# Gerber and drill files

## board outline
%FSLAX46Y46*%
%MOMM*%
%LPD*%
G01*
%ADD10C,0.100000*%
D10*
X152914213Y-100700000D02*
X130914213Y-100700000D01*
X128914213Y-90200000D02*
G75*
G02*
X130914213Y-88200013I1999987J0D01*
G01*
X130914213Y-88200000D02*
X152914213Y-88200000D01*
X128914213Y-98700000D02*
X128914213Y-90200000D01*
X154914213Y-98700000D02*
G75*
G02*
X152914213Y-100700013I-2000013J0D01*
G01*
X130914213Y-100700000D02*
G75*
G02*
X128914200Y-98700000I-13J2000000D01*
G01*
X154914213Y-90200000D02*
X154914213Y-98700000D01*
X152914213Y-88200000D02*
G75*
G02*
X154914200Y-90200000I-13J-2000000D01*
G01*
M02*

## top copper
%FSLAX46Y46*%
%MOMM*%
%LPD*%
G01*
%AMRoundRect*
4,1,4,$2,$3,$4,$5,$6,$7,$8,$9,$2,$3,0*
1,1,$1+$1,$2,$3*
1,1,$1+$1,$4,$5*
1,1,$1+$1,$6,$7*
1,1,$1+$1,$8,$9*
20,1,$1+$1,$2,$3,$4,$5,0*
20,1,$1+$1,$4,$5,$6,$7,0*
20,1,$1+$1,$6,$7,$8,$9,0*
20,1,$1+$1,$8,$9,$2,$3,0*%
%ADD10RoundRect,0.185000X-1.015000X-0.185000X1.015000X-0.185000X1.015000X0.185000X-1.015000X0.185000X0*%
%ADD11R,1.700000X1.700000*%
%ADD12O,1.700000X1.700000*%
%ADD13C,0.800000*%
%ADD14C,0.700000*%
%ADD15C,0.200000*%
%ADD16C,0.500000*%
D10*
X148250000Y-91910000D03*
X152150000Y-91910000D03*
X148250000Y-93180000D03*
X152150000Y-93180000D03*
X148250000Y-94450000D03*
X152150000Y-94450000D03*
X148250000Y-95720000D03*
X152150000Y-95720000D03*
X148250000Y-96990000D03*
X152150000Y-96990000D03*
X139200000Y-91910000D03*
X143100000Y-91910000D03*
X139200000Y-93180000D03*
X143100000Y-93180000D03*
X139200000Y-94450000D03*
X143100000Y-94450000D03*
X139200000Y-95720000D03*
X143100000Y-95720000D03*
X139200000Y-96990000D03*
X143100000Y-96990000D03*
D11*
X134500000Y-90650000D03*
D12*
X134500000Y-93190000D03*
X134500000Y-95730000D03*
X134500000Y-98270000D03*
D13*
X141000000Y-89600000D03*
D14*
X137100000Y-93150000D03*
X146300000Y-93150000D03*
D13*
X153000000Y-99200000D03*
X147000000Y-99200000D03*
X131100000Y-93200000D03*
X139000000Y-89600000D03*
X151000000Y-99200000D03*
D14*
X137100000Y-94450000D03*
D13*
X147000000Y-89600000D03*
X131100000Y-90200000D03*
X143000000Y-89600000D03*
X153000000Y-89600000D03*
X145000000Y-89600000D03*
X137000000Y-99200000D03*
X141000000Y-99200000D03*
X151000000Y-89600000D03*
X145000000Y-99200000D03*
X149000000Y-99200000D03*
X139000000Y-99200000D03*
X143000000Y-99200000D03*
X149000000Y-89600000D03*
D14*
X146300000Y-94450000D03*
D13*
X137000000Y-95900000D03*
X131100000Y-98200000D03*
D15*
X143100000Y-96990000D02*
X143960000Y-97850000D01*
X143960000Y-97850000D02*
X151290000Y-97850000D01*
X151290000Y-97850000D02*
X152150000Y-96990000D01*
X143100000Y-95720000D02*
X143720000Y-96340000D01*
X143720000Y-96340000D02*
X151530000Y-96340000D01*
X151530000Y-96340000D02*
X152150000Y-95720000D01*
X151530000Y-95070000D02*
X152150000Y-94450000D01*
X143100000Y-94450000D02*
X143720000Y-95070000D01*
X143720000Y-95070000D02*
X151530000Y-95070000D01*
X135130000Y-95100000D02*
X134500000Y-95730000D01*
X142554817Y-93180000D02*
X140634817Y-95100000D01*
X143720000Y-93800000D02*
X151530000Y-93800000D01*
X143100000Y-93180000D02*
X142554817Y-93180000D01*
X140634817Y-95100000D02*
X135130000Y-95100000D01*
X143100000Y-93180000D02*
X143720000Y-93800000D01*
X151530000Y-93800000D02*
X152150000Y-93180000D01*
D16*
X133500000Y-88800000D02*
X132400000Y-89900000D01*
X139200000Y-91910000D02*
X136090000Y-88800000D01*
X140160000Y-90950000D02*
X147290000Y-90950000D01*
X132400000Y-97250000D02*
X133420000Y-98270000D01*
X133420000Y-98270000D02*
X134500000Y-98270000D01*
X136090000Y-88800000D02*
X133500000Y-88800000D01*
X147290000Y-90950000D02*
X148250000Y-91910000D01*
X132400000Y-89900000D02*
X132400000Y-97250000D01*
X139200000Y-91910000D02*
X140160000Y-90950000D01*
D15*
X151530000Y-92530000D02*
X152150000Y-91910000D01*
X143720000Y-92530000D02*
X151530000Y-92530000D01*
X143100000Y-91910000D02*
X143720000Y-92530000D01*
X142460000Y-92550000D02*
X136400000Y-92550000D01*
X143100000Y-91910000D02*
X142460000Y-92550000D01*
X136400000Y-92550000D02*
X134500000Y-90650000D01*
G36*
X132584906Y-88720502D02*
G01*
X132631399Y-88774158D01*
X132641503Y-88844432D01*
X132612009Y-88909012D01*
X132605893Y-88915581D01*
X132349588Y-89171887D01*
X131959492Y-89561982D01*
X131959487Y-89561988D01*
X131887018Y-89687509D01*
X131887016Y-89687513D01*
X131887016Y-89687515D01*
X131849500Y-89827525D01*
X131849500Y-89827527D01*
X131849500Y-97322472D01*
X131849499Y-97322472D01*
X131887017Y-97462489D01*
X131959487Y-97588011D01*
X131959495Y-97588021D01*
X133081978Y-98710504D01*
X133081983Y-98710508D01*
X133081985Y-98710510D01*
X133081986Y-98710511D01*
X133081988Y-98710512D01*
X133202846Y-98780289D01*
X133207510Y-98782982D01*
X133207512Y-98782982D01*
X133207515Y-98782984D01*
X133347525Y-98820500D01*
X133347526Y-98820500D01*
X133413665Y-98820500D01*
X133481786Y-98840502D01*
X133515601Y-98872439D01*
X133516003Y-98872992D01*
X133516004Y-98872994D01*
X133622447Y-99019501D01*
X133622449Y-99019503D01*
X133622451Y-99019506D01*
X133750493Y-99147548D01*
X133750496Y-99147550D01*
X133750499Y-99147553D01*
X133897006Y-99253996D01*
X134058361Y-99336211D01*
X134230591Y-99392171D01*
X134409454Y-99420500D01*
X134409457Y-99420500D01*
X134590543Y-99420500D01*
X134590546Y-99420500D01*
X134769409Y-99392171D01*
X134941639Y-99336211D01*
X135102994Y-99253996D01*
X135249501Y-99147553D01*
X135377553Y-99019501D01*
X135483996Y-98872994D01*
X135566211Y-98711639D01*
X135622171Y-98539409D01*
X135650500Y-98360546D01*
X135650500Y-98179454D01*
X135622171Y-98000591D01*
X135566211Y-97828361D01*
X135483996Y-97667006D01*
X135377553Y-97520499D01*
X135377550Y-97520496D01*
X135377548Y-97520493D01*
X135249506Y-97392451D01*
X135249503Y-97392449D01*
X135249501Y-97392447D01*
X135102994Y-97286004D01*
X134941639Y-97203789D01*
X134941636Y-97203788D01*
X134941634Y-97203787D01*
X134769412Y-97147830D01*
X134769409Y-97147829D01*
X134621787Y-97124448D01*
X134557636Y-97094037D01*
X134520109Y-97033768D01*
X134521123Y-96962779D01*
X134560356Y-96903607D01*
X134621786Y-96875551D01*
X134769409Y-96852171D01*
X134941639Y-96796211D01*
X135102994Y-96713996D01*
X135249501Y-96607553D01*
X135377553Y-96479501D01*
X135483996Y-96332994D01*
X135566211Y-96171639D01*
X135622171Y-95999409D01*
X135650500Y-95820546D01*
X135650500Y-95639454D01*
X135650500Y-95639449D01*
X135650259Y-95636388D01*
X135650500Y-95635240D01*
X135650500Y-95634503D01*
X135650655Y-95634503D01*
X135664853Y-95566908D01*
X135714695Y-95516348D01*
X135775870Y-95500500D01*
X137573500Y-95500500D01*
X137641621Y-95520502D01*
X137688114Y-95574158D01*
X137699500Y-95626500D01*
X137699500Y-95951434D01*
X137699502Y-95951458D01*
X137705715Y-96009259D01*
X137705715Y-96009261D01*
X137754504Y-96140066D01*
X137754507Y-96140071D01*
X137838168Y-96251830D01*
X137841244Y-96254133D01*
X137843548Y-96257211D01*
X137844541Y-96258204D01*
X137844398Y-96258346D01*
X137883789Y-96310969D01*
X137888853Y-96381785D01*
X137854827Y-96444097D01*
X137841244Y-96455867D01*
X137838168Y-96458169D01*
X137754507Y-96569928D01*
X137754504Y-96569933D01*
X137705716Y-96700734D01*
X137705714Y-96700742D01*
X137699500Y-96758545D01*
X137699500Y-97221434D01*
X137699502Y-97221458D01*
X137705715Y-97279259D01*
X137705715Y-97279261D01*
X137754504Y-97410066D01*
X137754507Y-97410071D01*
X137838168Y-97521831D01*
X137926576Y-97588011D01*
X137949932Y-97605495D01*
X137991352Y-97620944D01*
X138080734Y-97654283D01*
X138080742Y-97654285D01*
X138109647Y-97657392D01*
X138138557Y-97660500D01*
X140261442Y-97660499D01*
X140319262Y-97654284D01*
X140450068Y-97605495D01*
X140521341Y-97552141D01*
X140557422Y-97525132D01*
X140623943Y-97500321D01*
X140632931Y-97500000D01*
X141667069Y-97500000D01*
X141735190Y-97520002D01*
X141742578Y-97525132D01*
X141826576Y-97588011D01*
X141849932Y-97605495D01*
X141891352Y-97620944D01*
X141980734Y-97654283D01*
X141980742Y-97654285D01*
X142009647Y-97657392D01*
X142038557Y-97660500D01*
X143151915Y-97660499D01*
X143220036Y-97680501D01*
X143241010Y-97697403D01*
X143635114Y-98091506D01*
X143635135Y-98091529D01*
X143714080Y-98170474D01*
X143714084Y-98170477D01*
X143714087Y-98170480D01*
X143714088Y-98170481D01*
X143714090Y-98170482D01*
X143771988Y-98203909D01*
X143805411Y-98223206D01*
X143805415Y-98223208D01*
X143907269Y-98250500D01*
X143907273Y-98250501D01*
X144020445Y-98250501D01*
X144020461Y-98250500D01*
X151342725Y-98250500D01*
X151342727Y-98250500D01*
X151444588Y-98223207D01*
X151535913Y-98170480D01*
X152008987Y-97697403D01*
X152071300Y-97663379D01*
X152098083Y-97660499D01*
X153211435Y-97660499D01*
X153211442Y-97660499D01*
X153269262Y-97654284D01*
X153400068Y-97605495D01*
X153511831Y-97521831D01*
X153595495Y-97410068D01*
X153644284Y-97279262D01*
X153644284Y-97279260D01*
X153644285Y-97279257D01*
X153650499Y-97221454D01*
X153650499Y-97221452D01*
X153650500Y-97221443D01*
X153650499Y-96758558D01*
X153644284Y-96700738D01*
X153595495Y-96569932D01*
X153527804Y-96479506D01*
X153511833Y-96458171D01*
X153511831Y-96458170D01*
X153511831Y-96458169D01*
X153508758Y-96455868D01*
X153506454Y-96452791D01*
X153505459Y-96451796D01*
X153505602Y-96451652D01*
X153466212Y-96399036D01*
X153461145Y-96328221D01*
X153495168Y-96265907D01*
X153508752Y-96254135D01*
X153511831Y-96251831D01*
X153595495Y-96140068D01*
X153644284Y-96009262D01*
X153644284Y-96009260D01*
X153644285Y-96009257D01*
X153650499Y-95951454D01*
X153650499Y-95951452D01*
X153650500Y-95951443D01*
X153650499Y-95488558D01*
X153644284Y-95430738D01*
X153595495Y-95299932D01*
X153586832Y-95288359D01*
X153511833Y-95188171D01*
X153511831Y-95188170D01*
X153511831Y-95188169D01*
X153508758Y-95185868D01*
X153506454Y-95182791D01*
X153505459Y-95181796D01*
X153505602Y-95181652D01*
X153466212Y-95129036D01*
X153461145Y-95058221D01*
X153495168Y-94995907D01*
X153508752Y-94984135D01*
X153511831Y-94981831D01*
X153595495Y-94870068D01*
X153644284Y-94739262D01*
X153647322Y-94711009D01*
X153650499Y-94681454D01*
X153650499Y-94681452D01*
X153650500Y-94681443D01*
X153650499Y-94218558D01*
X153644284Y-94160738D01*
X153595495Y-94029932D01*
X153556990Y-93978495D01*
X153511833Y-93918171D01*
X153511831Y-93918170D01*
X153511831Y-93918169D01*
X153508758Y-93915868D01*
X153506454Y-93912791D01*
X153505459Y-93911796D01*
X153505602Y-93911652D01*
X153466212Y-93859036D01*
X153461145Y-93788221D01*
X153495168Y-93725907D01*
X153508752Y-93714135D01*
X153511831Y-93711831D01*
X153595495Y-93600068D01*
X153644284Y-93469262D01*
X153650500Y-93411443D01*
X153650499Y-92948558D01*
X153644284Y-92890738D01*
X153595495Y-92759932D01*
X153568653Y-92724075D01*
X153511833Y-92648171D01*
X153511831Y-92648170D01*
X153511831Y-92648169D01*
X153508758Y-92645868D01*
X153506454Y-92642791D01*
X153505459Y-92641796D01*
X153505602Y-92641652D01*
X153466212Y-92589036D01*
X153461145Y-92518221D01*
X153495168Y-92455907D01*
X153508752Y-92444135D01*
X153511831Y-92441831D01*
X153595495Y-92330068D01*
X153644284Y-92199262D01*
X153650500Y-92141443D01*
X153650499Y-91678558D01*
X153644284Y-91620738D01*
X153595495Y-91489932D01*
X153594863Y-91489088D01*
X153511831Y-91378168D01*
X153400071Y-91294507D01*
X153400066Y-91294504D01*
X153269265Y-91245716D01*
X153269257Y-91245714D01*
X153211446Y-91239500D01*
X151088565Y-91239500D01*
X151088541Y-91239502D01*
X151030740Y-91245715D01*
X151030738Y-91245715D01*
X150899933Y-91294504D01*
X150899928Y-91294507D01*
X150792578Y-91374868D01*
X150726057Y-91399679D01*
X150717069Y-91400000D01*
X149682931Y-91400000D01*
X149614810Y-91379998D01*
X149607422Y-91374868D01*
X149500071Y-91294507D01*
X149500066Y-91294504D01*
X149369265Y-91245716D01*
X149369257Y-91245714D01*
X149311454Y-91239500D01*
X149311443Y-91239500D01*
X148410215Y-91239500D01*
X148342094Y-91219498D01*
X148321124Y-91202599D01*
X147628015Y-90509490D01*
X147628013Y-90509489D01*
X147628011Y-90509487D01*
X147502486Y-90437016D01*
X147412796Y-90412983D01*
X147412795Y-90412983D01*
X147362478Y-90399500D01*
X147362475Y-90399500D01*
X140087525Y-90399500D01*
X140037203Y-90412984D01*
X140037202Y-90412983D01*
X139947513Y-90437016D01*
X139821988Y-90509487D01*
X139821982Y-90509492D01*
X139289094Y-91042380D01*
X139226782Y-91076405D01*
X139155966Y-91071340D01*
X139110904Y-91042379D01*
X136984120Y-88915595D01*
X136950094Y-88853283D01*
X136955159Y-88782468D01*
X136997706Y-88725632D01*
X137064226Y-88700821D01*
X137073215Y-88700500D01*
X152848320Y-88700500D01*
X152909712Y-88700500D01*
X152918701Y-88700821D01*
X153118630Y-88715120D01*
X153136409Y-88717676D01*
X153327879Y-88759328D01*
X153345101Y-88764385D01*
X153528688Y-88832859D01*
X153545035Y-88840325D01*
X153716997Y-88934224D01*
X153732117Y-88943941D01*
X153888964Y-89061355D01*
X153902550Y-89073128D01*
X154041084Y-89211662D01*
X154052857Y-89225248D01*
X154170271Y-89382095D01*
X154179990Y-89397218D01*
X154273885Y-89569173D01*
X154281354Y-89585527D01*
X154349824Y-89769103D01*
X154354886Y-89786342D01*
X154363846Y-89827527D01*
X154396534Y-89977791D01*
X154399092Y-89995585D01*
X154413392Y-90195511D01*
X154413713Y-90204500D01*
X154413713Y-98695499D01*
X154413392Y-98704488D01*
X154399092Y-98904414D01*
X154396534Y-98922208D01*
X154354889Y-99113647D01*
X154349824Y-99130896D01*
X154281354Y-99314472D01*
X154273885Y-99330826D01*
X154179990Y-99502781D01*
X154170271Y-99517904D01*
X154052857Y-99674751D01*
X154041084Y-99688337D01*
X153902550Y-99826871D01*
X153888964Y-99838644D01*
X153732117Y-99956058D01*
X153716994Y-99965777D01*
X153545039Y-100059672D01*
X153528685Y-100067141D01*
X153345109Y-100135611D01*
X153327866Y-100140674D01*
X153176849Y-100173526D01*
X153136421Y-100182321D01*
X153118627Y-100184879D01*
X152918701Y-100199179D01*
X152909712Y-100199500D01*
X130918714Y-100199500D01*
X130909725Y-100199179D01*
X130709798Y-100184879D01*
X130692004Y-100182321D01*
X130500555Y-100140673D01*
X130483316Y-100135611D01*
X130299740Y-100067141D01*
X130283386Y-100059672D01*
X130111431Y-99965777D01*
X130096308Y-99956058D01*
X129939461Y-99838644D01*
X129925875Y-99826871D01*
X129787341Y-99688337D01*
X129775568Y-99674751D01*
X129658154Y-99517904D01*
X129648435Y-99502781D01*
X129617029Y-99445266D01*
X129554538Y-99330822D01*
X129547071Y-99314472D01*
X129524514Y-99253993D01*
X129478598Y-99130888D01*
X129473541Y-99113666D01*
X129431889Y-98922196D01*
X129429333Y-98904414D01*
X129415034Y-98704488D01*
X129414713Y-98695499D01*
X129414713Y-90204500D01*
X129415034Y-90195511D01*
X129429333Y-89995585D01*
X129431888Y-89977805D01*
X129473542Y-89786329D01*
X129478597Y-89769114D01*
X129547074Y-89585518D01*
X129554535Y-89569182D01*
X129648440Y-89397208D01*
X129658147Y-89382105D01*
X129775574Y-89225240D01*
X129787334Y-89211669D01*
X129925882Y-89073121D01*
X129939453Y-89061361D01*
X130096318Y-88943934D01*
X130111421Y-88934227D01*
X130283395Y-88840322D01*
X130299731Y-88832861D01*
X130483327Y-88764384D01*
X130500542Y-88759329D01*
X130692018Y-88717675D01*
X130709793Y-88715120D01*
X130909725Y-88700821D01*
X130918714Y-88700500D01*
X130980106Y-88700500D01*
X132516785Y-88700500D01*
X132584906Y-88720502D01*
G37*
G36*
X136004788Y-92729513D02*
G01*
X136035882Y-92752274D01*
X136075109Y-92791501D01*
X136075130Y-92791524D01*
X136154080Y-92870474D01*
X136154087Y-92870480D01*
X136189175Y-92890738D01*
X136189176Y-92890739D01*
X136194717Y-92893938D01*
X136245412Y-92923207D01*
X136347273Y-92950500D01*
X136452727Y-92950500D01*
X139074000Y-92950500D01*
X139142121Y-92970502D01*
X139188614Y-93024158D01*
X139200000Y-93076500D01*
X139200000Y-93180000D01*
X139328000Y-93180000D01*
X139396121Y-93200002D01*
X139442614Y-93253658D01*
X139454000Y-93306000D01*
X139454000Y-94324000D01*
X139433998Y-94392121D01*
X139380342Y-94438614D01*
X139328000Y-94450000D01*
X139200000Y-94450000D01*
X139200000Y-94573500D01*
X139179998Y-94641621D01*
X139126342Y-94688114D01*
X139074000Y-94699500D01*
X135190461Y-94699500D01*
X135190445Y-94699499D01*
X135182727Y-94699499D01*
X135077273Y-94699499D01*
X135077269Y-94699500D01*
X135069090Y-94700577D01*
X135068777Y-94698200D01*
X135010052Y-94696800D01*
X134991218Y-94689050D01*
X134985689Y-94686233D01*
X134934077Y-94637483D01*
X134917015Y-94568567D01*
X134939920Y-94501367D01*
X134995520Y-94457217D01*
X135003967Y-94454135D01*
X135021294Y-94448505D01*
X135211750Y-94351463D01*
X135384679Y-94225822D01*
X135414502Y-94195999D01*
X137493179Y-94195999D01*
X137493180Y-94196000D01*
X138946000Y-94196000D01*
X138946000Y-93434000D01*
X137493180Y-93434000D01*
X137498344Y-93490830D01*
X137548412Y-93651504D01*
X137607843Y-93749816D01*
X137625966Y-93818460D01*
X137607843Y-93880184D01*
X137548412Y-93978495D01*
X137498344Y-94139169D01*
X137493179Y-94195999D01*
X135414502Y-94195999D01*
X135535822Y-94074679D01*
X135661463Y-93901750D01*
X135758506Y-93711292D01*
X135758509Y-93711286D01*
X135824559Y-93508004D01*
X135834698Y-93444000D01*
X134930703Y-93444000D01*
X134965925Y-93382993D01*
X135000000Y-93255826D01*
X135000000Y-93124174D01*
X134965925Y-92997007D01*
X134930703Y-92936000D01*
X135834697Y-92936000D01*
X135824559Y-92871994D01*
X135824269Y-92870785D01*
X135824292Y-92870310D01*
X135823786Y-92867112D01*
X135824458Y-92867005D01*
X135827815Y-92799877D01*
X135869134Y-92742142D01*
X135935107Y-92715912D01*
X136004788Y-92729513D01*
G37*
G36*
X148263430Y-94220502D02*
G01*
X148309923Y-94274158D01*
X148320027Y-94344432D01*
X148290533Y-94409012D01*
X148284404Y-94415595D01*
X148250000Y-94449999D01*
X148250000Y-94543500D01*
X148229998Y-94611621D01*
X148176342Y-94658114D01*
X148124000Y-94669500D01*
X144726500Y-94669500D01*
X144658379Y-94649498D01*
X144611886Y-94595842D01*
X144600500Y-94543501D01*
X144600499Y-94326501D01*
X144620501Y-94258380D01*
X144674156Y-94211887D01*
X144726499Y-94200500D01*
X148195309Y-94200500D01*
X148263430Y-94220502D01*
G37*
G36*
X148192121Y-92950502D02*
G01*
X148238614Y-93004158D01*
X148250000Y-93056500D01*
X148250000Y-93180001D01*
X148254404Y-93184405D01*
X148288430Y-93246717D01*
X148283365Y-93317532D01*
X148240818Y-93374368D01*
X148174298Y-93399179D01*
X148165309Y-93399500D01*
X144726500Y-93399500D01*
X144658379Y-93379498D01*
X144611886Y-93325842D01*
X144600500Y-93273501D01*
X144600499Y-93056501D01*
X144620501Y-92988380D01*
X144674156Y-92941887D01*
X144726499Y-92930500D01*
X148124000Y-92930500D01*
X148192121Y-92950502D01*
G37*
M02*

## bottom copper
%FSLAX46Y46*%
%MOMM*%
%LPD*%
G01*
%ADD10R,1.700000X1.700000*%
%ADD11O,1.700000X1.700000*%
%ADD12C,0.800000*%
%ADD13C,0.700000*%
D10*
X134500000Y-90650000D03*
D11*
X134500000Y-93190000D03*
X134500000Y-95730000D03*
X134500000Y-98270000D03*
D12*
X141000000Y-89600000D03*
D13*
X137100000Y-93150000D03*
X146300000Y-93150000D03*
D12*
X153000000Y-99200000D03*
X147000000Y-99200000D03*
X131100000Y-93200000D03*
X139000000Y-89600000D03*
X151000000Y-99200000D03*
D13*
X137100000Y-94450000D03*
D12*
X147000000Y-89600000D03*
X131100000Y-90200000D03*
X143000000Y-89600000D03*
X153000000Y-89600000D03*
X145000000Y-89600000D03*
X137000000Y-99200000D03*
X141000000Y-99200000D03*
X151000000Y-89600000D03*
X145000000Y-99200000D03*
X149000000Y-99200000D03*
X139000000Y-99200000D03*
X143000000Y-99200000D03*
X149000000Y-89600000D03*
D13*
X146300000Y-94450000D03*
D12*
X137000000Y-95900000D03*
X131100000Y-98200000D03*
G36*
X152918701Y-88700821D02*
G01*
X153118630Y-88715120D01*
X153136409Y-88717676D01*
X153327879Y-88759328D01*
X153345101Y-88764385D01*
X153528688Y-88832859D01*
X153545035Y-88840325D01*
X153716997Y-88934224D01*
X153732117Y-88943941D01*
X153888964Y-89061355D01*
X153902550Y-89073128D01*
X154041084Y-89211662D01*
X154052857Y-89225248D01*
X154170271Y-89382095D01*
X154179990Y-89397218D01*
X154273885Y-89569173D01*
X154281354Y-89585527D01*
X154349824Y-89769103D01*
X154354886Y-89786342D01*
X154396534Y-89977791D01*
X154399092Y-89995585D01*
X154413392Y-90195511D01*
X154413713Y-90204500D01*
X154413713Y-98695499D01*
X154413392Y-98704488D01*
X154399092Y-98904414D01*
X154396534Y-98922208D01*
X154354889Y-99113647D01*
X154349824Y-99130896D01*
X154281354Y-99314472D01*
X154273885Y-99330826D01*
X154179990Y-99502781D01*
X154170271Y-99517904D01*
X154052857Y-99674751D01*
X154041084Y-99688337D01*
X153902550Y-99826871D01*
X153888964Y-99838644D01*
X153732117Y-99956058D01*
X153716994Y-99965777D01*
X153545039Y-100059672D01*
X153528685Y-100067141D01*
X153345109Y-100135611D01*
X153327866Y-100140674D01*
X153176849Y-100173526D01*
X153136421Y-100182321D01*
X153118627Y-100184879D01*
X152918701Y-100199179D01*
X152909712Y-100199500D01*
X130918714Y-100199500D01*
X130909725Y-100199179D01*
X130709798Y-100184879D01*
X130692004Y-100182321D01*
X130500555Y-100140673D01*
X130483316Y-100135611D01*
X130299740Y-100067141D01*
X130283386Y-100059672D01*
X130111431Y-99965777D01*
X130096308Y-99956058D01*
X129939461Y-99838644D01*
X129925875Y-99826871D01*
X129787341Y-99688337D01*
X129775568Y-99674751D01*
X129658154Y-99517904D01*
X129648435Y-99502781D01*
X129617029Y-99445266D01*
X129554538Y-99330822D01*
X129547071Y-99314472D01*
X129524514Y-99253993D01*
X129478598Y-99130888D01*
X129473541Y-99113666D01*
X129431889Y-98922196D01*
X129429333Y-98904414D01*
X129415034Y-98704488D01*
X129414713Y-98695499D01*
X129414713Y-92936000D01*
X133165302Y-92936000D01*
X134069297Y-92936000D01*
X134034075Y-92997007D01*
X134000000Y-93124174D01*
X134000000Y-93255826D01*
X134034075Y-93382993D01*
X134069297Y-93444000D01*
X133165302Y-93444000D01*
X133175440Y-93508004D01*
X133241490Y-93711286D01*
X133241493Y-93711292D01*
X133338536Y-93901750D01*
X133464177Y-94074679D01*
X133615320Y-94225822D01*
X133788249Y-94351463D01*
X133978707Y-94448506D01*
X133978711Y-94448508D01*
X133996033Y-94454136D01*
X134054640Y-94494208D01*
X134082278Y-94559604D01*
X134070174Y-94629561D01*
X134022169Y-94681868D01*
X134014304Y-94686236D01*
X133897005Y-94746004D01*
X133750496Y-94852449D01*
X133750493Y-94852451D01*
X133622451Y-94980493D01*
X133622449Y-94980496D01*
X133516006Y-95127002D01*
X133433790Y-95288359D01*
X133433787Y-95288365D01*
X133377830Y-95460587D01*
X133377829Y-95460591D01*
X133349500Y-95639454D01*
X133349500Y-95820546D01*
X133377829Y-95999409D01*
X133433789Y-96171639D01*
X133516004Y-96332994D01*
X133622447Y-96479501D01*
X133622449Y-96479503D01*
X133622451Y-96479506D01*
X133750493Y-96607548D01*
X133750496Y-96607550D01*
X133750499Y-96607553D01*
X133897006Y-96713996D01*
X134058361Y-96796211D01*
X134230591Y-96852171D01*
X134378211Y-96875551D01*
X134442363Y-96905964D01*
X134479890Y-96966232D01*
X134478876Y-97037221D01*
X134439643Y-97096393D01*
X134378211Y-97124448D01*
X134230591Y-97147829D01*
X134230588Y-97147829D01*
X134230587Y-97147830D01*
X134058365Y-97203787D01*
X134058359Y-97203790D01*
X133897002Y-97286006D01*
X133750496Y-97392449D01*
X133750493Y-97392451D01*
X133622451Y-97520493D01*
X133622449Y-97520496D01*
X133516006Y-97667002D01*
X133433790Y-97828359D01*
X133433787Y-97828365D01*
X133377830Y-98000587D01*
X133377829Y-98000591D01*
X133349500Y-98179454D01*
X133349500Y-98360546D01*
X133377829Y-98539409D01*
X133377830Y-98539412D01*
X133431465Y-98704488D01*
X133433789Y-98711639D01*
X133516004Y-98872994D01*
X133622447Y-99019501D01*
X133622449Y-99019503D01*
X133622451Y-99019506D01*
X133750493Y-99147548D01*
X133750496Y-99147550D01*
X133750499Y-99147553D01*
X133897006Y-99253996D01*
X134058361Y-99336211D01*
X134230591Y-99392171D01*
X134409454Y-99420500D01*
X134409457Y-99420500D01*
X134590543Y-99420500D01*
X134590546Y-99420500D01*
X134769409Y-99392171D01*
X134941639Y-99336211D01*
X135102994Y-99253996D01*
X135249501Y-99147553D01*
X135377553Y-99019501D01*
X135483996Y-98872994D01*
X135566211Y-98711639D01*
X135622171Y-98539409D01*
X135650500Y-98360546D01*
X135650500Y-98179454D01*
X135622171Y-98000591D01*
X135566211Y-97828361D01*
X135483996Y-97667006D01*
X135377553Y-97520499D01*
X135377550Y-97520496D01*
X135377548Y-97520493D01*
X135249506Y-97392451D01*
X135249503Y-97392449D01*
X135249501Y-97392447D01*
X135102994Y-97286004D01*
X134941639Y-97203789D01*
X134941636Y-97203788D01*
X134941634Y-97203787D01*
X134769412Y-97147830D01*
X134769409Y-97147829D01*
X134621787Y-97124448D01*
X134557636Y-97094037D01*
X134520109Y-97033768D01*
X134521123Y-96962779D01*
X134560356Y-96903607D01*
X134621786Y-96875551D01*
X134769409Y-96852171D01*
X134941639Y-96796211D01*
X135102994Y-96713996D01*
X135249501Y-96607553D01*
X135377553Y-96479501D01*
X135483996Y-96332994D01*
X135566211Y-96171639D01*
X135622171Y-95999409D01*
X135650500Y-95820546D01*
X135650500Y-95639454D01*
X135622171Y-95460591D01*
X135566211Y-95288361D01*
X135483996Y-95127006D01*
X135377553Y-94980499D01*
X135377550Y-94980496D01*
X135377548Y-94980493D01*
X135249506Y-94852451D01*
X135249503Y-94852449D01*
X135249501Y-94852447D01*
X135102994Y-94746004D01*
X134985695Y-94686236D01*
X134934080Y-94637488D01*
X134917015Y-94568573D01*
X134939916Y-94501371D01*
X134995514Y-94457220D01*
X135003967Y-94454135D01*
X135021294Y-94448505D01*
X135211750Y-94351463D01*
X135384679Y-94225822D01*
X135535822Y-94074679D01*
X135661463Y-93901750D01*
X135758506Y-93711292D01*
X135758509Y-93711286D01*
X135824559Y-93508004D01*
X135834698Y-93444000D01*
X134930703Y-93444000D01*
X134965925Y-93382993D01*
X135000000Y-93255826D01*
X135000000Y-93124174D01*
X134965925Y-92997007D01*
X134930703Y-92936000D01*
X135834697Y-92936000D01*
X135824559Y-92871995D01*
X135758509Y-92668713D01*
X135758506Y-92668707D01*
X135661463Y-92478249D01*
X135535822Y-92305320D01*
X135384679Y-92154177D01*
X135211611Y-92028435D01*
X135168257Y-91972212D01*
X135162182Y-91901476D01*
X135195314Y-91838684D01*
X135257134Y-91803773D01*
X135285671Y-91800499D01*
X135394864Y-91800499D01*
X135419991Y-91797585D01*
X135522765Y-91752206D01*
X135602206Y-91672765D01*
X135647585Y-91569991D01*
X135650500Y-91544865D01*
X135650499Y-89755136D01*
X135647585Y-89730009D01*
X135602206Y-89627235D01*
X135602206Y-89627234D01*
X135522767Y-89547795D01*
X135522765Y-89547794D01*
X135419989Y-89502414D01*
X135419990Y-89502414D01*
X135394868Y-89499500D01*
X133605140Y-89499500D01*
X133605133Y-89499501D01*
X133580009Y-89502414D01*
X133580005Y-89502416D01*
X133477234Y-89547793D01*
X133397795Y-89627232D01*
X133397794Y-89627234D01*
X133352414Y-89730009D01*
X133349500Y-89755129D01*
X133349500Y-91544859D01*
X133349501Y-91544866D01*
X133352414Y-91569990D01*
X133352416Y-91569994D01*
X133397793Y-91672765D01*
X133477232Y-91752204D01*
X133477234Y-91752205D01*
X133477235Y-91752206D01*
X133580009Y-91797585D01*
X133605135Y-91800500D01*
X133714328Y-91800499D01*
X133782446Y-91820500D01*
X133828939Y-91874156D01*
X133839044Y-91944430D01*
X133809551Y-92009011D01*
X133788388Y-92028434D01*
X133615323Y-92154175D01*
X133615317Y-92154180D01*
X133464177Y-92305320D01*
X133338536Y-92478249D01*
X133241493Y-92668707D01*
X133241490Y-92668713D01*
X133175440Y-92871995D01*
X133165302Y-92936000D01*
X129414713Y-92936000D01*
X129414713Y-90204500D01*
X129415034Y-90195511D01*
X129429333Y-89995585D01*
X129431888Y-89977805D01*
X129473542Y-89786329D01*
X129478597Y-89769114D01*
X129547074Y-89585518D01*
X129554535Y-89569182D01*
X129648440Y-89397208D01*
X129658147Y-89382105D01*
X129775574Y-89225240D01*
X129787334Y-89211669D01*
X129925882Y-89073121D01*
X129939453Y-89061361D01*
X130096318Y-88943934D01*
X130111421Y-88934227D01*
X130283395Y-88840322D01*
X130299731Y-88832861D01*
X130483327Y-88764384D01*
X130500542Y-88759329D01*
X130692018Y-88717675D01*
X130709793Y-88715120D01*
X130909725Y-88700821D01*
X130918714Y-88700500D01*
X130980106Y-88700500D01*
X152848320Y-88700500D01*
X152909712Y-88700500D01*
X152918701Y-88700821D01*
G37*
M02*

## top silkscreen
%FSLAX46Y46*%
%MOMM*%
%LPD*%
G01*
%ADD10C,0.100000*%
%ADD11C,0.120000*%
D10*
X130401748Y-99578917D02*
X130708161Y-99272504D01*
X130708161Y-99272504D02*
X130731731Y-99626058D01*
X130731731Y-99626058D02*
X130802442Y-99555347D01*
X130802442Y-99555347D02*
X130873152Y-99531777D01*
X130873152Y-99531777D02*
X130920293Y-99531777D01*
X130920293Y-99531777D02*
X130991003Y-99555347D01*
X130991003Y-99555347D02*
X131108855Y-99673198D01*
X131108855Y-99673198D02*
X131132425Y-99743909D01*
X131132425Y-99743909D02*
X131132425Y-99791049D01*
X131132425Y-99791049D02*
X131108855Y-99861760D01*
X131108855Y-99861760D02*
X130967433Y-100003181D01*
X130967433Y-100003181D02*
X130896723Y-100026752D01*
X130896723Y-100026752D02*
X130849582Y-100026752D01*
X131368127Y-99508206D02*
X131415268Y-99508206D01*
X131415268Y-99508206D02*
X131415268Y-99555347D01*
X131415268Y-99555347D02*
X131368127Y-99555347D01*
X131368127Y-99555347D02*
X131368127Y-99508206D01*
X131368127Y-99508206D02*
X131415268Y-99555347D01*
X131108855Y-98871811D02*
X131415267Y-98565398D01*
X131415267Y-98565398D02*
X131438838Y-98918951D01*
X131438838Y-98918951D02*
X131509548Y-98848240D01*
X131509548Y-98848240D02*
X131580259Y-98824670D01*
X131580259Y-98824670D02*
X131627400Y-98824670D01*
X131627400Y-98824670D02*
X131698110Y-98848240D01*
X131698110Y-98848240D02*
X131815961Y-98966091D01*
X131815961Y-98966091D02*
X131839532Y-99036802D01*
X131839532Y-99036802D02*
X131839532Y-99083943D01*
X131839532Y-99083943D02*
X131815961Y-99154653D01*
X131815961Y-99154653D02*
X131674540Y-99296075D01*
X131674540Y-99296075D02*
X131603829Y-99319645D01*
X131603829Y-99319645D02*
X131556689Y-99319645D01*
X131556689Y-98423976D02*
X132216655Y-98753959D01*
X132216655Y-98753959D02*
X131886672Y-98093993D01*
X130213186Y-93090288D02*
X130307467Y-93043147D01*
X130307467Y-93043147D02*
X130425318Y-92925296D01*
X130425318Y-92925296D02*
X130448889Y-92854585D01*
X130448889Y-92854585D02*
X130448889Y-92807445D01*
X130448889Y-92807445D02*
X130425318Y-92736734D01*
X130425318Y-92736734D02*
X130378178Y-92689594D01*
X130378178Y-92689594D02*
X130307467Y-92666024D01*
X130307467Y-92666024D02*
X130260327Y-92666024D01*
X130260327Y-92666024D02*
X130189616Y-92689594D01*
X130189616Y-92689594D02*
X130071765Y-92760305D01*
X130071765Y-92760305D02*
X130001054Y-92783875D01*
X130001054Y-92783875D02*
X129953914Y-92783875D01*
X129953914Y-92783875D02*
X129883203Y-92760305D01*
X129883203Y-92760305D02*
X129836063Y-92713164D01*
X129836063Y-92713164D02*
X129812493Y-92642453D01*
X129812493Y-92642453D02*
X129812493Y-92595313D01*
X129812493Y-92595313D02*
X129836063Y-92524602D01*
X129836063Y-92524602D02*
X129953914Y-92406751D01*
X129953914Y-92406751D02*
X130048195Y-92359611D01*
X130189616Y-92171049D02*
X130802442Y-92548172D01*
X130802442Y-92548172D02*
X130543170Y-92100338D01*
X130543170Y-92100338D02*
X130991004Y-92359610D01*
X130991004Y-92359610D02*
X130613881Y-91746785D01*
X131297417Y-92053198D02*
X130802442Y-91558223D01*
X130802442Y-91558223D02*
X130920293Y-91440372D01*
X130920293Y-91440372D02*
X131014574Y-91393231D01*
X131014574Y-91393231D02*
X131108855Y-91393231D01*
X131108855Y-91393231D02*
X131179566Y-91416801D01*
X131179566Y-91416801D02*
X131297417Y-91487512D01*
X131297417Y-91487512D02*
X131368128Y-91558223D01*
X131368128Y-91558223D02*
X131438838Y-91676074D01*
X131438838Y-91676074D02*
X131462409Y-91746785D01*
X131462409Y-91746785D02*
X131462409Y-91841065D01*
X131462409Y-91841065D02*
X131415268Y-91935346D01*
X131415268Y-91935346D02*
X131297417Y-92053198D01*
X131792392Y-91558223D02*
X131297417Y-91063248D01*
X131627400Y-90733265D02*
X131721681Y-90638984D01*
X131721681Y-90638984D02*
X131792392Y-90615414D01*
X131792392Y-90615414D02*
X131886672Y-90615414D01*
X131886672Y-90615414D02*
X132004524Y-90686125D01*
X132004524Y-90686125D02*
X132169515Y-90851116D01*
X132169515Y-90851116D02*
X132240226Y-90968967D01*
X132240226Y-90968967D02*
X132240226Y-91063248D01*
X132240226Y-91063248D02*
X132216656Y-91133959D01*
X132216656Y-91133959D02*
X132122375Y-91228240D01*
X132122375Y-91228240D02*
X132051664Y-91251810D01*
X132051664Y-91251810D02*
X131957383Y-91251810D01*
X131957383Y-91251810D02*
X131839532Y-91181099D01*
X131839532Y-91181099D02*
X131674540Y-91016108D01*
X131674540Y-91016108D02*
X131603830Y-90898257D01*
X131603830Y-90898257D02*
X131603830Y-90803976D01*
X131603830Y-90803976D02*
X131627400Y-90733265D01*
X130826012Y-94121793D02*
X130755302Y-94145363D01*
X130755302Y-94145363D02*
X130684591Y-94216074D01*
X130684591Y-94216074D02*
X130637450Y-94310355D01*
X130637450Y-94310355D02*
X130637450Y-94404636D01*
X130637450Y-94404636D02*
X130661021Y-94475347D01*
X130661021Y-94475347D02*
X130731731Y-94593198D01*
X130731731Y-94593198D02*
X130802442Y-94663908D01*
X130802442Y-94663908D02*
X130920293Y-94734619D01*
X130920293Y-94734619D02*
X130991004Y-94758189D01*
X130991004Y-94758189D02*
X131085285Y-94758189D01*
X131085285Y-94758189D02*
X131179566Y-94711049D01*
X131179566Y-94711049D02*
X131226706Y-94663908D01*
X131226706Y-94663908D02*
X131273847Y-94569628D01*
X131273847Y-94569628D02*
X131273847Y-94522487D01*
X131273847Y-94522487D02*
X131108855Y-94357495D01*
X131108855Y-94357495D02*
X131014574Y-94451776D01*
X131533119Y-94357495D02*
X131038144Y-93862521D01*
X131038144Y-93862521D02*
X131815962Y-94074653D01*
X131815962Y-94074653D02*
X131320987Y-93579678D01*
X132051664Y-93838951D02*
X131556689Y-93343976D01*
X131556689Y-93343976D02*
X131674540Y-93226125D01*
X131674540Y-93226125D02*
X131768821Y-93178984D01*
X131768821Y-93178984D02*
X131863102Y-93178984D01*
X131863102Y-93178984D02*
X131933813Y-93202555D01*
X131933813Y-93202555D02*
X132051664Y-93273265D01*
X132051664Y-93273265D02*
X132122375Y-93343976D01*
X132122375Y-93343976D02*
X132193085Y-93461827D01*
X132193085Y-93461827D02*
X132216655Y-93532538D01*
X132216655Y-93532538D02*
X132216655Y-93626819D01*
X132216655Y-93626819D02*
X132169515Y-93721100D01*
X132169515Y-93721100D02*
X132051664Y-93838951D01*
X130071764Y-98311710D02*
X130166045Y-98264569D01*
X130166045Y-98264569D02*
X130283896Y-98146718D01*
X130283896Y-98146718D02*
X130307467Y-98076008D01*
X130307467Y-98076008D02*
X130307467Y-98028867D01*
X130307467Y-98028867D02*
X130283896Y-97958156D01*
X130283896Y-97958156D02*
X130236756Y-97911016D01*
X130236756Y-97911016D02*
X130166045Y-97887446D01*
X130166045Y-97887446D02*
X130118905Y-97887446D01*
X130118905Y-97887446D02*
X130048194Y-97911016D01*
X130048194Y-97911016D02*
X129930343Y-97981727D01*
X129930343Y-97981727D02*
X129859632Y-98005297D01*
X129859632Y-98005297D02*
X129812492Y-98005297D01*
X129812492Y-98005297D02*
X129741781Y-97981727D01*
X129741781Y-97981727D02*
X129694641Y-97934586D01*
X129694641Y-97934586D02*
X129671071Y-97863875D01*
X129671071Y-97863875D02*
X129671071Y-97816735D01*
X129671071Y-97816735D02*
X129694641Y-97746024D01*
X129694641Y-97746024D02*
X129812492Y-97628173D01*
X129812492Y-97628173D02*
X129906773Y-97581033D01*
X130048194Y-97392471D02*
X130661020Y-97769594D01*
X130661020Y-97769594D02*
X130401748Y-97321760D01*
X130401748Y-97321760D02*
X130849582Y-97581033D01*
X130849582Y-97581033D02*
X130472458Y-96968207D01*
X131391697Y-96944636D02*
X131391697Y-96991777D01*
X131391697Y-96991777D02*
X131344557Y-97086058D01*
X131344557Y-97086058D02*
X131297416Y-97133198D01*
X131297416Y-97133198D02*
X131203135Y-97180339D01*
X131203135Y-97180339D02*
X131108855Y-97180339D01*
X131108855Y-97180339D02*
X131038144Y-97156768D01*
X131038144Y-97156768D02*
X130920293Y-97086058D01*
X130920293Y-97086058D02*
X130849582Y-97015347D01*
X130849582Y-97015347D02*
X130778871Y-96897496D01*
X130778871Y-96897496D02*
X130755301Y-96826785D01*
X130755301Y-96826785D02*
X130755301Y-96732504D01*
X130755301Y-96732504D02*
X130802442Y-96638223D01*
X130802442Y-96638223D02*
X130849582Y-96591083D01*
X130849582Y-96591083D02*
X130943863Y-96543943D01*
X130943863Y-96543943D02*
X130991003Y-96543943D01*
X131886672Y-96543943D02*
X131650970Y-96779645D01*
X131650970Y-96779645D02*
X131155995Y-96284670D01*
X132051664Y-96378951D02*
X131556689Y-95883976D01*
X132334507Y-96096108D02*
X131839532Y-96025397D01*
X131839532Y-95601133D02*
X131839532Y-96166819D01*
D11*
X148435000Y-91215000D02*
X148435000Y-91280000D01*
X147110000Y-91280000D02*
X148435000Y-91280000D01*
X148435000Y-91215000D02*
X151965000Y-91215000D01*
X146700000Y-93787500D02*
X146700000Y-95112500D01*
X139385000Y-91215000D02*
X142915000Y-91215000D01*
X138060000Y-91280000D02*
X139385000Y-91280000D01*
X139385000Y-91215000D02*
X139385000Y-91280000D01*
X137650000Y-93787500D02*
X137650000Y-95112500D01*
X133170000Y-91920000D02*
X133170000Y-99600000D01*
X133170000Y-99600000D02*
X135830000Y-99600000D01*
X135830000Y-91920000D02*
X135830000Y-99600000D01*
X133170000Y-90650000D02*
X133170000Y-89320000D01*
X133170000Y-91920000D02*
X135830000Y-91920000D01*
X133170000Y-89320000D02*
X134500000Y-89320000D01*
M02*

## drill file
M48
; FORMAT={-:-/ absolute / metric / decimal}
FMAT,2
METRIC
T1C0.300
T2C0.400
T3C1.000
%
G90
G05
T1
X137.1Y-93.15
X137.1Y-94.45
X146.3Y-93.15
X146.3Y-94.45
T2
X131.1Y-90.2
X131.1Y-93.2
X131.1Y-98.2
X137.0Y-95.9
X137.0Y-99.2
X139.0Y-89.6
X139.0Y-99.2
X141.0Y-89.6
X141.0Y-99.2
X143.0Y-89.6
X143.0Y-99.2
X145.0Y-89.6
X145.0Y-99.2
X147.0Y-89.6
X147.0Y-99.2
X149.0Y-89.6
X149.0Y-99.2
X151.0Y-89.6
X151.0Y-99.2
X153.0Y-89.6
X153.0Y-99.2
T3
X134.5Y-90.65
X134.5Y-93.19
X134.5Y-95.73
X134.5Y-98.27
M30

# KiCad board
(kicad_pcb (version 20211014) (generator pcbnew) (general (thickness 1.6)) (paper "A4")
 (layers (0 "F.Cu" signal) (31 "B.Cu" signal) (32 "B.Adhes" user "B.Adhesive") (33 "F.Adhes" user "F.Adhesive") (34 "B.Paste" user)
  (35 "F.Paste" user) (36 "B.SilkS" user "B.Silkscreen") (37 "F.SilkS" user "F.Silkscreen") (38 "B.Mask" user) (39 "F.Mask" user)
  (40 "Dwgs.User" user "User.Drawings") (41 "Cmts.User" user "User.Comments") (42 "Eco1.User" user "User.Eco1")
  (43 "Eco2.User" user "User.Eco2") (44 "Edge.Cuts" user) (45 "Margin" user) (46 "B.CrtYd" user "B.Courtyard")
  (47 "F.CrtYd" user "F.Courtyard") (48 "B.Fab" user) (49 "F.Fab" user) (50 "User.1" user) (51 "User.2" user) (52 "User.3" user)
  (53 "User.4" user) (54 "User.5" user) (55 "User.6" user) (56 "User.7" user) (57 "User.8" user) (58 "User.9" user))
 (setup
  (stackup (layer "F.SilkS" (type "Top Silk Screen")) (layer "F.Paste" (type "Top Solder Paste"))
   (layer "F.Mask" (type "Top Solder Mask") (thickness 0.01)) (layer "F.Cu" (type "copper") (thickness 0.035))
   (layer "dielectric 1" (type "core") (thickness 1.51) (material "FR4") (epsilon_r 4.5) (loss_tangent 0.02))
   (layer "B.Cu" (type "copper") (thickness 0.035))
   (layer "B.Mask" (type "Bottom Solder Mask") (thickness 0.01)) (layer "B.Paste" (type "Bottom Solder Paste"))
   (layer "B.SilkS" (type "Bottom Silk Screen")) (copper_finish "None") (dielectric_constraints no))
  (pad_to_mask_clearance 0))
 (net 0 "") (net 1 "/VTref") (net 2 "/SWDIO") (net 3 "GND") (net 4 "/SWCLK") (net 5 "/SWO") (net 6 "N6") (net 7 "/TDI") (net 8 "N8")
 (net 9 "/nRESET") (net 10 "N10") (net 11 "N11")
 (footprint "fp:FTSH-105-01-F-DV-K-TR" (layer "F.Cu") (at 150.2 94.45)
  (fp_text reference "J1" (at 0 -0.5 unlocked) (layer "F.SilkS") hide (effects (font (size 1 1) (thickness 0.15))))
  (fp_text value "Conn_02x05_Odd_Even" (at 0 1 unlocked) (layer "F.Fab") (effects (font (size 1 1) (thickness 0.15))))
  (fp_line (start -1.765 -3.235) (end -1.765 -3.17) (layer "F.SilkS") (width 0.12))
  (fp_line (start -3.09 -3.17) (end -1.765 -3.17) (layer "F.SilkS") (width 0.12))
  (fp_line (start -1.765 -3.235) (end 1.765 -3.235) (layer "F.SilkS") (width 0.12))
  (fp_line (start -3.5 -0.6625) (end -3.5 0.6625) (layer "F.SilkS") (width 0.12))
  (pad "1" smd roundrect (at -1.95 -2.54) (size 2.4 0.74) (layers "F.Cu" "F.Paste" "F.Mask") (roundrect_rratio 0.25) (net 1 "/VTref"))
  (pad "2" smd roundrect (at 1.95 -2.54) (size 2.4 0.74) (layers "F.Cu" "F.Paste" "F.Mask") (roundrect_rratio 0.25) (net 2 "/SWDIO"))
  (pad "3" smd roundrect (at -1.95 -1.27) (size 2.4 0.74) (layers "F.Cu" "F.Paste" "F.Mask") (roundrect_rratio 0.25) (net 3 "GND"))
  (pad "4" smd roundrect (at 1.95 -1.27) (size 2.4 0.74) (layers "F.Cu" "F.Paste" "F.Mask") (roundrect_rratio 0.25) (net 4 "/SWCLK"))
  (pad "5" smd roundrect (at -1.95 0) (size 2.4 0.74) (layers "F.Cu" "F.Paste" "F.Mask") (roundrect_rratio 0.25) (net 3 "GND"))
  (pad "6" smd roundrect (at 1.95 0) (size 2.4 0.74) (layers "F.Cu" "F.Paste" "F.Mask") (roundrect_rratio 0.25) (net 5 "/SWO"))
  (pad "7" smd roundrect (at -1.95 1.27) (size 2.4 0.74) (layers "F.Cu" "F.Paste" "F.Mask") (roundrect_rratio 0.25) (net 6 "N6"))
  (pad "8" smd roundrect (at 1.95 1.27) (size 2.4 0.74) (layers "F.Cu" "F.Paste" "F.Mask") (roundrect_rratio 0.25) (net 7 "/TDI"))
  (pad "9" smd roundrect (at -1.95 2.54) (size 2.4 0.74) (layers "F.Cu" "F.Paste" "F.Mask") (roundrect_rratio 0.25) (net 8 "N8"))
  (pad "10" smd roundrect (at 1.95 2.54) (size 2.4 0.74) (layers "F.Cu" "F.Paste" "F.Mask") (roundrect_rratio 0.25) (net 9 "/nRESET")))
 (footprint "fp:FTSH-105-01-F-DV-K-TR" (layer "F.Cu") (at 141.15 94.45)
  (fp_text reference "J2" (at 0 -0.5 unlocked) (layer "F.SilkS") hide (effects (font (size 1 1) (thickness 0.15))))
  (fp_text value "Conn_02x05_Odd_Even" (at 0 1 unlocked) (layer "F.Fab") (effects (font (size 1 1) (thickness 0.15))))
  (fp_line (start -1.765 -3.235) (end 1.765 -3.235) (layer "F.SilkS") (width 0.12))
  (fp_line (start -3.09 -3.17) (end -1.765 -3.17) (layer "F.SilkS") (width 0.12))
  (fp_line (start -1.765 -3.235) (end -1.765 -3.17) (layer "F.SilkS") (width 0.12))
  (fp_line (start -3.5 -0.6625) (end -3.5 0.6625) (layer "F.SilkS") (width 0.12))
  (pad "1" smd roundrect (at -1.95 -2.54) (size 2.4 0.74) (layers "F.Cu" "F.Paste" "F.Mask") (roundrect_rratio 0.25) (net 1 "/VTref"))
  (pad "2" smd roundrect (at 1.95 -2.54) (size 2.4 0.74) (layers "F.Cu" "F.Paste" "F.Mask") (roundrect_rratio 0.25) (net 2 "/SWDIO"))
  (pad "3" smd roundrect (at -1.95 -1.27) (size 2.4 0.74) (layers "F.Cu" "F.Paste" "F.Mask") (roundrect_rratio 0.25) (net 3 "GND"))
  (pad "4" smd roundrect (at 1.95 -1.27) (size 2.4 0.74) (layers "F.Cu" "F.Paste" "F.Mask") (roundrect_rratio 0.25) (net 4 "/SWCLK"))
  (pad "5" smd roundrect (at -1.95 0) (size 2.4 0.74) (layers "F.Cu" "F.Paste" "F.Mask") (roundrect_rratio 0.25) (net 3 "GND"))
  (pad "6" smd roundrect (at 1.95 0) (size 2.4 0.74) (layers "F.Cu" "F.Paste" "F.Mask") (roundrect_rratio 0.25) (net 5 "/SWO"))
  (pad "7" smd roundrect (at -1.95 1.27) (size 2.4 0.74) (layers "F.Cu" "F.Paste" "F.Mask") (roundrect_rratio 0.25) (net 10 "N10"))
  (pad "8" smd roundrect (at 1.95 1.27) (size 2.4 0.74) (layers "F.Cu" "F.Paste" "F.Mask") (roundrect_rratio 0.25) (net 7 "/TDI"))
  (pad "9" smd roundrect (at -1.95 2.54) (size 2.4 0.74) (layers "F.Cu" "F.Paste" "F.Mask") (roundrect_rratio 0.25) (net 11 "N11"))
  (pad "10" smd roundrect (at 1.95 2.54) (size 2.4 0.74) (layers "F.Cu" "F.Paste" "F.Mask") (roundrect_rratio 0.25) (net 9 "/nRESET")))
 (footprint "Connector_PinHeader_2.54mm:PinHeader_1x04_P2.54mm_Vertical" (layer "F.Cu") (at 134.5 90.65)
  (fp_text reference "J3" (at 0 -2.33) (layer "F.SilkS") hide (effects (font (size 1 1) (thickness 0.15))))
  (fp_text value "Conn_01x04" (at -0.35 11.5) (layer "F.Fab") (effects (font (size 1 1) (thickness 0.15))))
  (fp_line (start -1.33 1.27) (end -1.33 8.95) (layer "F.SilkS") (width 0.12))
  (fp_line (start -1.33 8.95) (end 1.33 8.95) (layer "F.SilkS") (width 0.12))
  (fp_line (start 1.33 1.27) (end 1.33 8.95) (layer "F.SilkS") (width 0.12))
  (fp_line (start -1.33 0) (end -1.33 -1.33) (layer "F.SilkS") (width 0.12))
  (fp_line (start -1.33 1.27) (end 1.33 1.27) (layer "F.SilkS") (width 0.12))
  (fp_line (start -1.33 -1.33) (end 0 -1.33) (layer "F.SilkS") (width 0.12))
  (pad "1" thru_hole rect (at 0 0) (size 1.7 1.7) (drill 1) (layers *.Cu *.Mask) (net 2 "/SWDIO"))
  (pad "2" thru_hole oval (at 0 2.54) (size 1.7 1.7) (drill 1) (layers *.Cu *.Mask) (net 3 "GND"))
  (pad "3" thru_hole oval (at 0 5.08) (size 1.7 1.7) (drill 1) (layers *.Cu *.Mask) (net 4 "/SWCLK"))
  (pad "4" thru_hole oval (at 0 7.62) (size 1.7 1.7) (drill 1) (layers *.Cu *.Mask) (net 1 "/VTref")))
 (gr_line (start 152.914213 100.7) (end 130.914213 100.7) (layer "Edge.Cuts") (width 0.1))
 (gr_arc (start 128.914213 90.2) (mid 129.5 88.785787) (end 130.914213 88.2) (layer "Edge.Cuts") (width 0.1))
 (gr_line (start 130.914213 88.2) (end 152.914213 88.2) (layer "Edge.Cuts") (width 0.1))
 (gr_line (start 128.914213 98.7) (end 128.914213 90.2) (layer "Edge.Cuts") (width 0.1))
 (gr_arc (start 154.914213 98.7) (mid 154.328426 100.114213) (end 152.914213 100.7) (layer "Edge.Cuts") (width 0.1))
 (gr_arc (start 130.914213 100.7) (mid 129.5 100.114213) (end 128.914213 98.7) (layer "Edge.Cuts") (width 0.1))
 (gr_line (start 154.914213 90.2) (end 154.914213 98.7) (layer "Edge.Cuts") (width 0.1))
 (gr_arc (start 152.914213 88.2) (mid 154.328426 88.785787) (end 154.914213 90.2) (layer "Edge.Cuts") (width 0.1))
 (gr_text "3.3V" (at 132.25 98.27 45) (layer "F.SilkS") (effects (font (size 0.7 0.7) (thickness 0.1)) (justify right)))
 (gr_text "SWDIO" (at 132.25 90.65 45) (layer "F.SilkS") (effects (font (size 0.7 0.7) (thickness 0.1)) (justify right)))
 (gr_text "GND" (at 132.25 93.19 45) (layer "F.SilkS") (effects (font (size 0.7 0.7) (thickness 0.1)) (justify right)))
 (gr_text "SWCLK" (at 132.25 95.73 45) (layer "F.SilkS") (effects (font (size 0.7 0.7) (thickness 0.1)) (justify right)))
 (segment (start 143.1 96.99) (end 143.96 97.85) (width 0.2) (layer "F.Cu") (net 9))
 (segment (start 143.96 97.85) (end 151.29 97.85) (width 0.2) (layer "F.Cu") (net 9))
 (segment (start 151.29 97.85) (end 152.15 96.99) (width 0.2) (layer "F.Cu") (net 9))
 (segment (start 143.1 95.72) (end 143.72 96.34) (width 0.2) (layer "F.Cu") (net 7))
 (segment (start 143.72 96.34) (end 151.53 96.34) (width 0.2) (layer "F.Cu") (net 7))
 (segment (start 151.53 96.34) (end 152.15 95.72) (width 0.2) (layer "F.Cu") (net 7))
 (via (at 141 89.6) (size 0.8) (drill 0.4) (layers "F.Cu" "B.Cu") (free) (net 3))
 (via (at 137.1 93.15) (size 0.7) (drill 0.3) (layers "F.Cu" "B.Cu") (free) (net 3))
 (via (at 146.3 93.15) (size 0.7) (drill 0.3) (layers "F.Cu" "B.Cu") (free) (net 3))
 (via (at 153 99.2) (size 0.8) (drill 0.4) (layers "F.Cu" "B.Cu") (free) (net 3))
 (via (at 147 99.2) (size 0.8) (drill 0.4) (layers "F.Cu" "B.Cu") (free) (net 3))
 (via (at 131.1 93.2) (size 0.8) (drill 0.4) (layers "F.Cu" "B.Cu") (free) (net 3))
 (via (at 139 89.6) (size 0.8) (drill 0.4) (layers "F.Cu" "B.Cu") (free) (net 3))
 (via (at 151 99.2) (size 0.8) (drill 0.4) (layers "F.Cu" "B.Cu") (free) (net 3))
 (via (at 137.1 94.45) (size 0.7) (drill 0.3) (layers "F.Cu" "B.Cu") (free) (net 3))
 (via (at 147 89.6) (size 0.8) (drill 0.4) (layers "F.Cu" "B.Cu") (free) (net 3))
 (via (at 131.1 90.2) (size 0.8) (drill 0.4) (layers "F.Cu" "B.Cu") (free) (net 3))
 (via (at 143 89.6) (size 0.8) (drill 0.4) (layers "F.Cu" "B.Cu") (free) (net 3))
 (via (at 153 89.6) (size 0.8) (drill 0.4) (layers "F.Cu" "B.Cu") (free) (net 3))
 (via (at 145 89.6) (size 0.8) (drill 0.4) (layers "F.Cu" "B.Cu") (free) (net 3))
 (via (at 137 99.2) (size 0.8) (drill 0.4) (layers "F.Cu" "B.Cu") (free) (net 3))
 (via (at 141 99.2) (size 0.8) (drill 0.4) (layers "F.Cu" "B.Cu") (free) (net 3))
 (via (at 151 89.6) (size 0.8) (drill 0.4) (layers "F.Cu" "B.Cu") (free) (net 3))
 (via (at 145 99.2) (size 0.8) (drill 0.4) (layers "F.Cu" "B.Cu") (free) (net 3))
 (via (at 149 99.2) (size 0.8) (drill 0.4) (layers "F.Cu" "B.Cu") (free) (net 3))
 (via (at 139 99.2) (size 0.8) (drill 0.4) (layers "F.Cu" "B.Cu") (free) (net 3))
 (via (at 143 99.2) (size 0.8) (drill 0.4) (layers "F.Cu" "B.Cu") (free) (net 3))
 (via (at 149 89.6) (size 0.8) (drill 0.4) (layers "F.Cu" "B.Cu") (free) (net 3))
 (via (at 146.3 94.45) (size 0.7) (drill 0.3) (layers "F.Cu" "B.Cu") (free) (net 3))
 (via (at 137 95.9) (size 0.8) (drill 0.4) (layers "F.Cu" "B.Cu") (free) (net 3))
 (via (at 131.1 98.2) (size 0.8) (drill 0.4) (layers "F.Cu" "B.Cu") (free) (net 3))
 (segment (start 151.53 95.07) (end 152.15 94.45) (width 0.2) (layer "F.Cu") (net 5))
 (segment (start 143.1 94.45) (end 143.72 95.07) (width 0.2) (layer "F.Cu") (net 5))
 (segment (start 143.72 95.07) (end 151.53 95.07) (width 0.2) (layer "F.Cu") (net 5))
 (segment (start 135.13 95.1) (end 134.5 95.73) (width 0.2) (layer "F.Cu") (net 4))
 (segment (start 142.554817 93.18) (end 140.634817 95.1) (width 0.2) (layer "F.Cu") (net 4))
 (segment (start 143.72 93.8) (end 151.53 93.8) (width 0.2) (layer "F.Cu") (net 4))
 (segment (start 143.1 93.18) (end 142.554817 93.18) (width 0.2) (layer "F.Cu") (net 4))
 (segment (start 140.634817 95.1) (end 135.13 95.1) (width 0.2) (layer "F.Cu") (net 4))
 (segment (start 143.1 93.18) (end 143.72 93.8) (width 0.2) (layer "F.Cu") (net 4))
 (segment (start 151.53 93.8) (end 152.15 93.18) (width 0.2) (layer "F.Cu") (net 4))
 (segment (start 133.5 88.8) (end 132.4 89.9) (width 0.5) (layer "F.Cu") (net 1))
 (segment (start 139.2 91.91) (end 136.09 88.8) (width 0.5) (layer "F.Cu") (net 1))
 (segment (start 140.16 90.95) (end 147.29 90.95) (width 0.5) (layer "F.Cu") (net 1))
 (segment (start 132.4 97.25) (end 133.42 98.27) (width 0.5) (layer "F.Cu") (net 1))
 (segment (start 133.42 98.27) (end 134.5 98.27) (width 0.5) (layer "F.Cu") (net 1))
 (segment (start 136.09 88.8) (end 133.5 88.8) (width 0.5) (layer "F.Cu") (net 1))
 (segment (start 147.29 90.95) (end 148.25 91.91) (width 0.5) (layer "F.Cu") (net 1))
 (segment (start 132.4 89.9) (end 132.4 97.25) (width 0.5) (layer "F.Cu") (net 1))
 (segment (start 139.2 91.91) (end 140.16 90.95) (width 0.5) (layer "F.Cu") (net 1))
 (segment (start 151.53 92.53) (end 152.15 91.91) (width 0.2) (layer "F.Cu") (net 2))
 (segment (start 143.72 92.53) (end 151.53 92.53) (width 0.2) (layer "F.Cu") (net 2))
 (segment (start 143.1 91.91) (end 143.72 92.53) (width 0.2) (layer "F.Cu") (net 2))
 (segment (start 142.46 92.55) (end 136.4 92.55) (width 0.2) (layer "F.Cu") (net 2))
 (segment (start 143.1 91.91) (end 142.46 92.55) (width 0.2) (layer "F.Cu") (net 2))
 (segment (start 136.4 92.55) (end 134.5 90.65) (width 0.2) (layer "F.Cu") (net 2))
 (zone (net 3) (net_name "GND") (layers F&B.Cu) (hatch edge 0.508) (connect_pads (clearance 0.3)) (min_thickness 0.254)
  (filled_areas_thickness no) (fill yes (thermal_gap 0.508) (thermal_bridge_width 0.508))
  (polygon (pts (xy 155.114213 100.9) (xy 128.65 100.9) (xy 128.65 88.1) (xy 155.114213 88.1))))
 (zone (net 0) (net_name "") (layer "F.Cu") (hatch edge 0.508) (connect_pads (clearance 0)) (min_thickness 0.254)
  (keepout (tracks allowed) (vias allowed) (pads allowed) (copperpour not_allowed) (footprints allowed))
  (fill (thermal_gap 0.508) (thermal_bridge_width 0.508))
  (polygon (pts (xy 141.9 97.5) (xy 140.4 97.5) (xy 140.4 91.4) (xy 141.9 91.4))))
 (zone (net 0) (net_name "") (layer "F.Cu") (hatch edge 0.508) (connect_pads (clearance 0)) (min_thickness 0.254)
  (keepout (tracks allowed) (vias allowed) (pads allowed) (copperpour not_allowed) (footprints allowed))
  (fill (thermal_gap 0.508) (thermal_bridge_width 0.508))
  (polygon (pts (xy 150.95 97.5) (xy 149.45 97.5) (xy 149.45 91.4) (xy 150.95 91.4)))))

